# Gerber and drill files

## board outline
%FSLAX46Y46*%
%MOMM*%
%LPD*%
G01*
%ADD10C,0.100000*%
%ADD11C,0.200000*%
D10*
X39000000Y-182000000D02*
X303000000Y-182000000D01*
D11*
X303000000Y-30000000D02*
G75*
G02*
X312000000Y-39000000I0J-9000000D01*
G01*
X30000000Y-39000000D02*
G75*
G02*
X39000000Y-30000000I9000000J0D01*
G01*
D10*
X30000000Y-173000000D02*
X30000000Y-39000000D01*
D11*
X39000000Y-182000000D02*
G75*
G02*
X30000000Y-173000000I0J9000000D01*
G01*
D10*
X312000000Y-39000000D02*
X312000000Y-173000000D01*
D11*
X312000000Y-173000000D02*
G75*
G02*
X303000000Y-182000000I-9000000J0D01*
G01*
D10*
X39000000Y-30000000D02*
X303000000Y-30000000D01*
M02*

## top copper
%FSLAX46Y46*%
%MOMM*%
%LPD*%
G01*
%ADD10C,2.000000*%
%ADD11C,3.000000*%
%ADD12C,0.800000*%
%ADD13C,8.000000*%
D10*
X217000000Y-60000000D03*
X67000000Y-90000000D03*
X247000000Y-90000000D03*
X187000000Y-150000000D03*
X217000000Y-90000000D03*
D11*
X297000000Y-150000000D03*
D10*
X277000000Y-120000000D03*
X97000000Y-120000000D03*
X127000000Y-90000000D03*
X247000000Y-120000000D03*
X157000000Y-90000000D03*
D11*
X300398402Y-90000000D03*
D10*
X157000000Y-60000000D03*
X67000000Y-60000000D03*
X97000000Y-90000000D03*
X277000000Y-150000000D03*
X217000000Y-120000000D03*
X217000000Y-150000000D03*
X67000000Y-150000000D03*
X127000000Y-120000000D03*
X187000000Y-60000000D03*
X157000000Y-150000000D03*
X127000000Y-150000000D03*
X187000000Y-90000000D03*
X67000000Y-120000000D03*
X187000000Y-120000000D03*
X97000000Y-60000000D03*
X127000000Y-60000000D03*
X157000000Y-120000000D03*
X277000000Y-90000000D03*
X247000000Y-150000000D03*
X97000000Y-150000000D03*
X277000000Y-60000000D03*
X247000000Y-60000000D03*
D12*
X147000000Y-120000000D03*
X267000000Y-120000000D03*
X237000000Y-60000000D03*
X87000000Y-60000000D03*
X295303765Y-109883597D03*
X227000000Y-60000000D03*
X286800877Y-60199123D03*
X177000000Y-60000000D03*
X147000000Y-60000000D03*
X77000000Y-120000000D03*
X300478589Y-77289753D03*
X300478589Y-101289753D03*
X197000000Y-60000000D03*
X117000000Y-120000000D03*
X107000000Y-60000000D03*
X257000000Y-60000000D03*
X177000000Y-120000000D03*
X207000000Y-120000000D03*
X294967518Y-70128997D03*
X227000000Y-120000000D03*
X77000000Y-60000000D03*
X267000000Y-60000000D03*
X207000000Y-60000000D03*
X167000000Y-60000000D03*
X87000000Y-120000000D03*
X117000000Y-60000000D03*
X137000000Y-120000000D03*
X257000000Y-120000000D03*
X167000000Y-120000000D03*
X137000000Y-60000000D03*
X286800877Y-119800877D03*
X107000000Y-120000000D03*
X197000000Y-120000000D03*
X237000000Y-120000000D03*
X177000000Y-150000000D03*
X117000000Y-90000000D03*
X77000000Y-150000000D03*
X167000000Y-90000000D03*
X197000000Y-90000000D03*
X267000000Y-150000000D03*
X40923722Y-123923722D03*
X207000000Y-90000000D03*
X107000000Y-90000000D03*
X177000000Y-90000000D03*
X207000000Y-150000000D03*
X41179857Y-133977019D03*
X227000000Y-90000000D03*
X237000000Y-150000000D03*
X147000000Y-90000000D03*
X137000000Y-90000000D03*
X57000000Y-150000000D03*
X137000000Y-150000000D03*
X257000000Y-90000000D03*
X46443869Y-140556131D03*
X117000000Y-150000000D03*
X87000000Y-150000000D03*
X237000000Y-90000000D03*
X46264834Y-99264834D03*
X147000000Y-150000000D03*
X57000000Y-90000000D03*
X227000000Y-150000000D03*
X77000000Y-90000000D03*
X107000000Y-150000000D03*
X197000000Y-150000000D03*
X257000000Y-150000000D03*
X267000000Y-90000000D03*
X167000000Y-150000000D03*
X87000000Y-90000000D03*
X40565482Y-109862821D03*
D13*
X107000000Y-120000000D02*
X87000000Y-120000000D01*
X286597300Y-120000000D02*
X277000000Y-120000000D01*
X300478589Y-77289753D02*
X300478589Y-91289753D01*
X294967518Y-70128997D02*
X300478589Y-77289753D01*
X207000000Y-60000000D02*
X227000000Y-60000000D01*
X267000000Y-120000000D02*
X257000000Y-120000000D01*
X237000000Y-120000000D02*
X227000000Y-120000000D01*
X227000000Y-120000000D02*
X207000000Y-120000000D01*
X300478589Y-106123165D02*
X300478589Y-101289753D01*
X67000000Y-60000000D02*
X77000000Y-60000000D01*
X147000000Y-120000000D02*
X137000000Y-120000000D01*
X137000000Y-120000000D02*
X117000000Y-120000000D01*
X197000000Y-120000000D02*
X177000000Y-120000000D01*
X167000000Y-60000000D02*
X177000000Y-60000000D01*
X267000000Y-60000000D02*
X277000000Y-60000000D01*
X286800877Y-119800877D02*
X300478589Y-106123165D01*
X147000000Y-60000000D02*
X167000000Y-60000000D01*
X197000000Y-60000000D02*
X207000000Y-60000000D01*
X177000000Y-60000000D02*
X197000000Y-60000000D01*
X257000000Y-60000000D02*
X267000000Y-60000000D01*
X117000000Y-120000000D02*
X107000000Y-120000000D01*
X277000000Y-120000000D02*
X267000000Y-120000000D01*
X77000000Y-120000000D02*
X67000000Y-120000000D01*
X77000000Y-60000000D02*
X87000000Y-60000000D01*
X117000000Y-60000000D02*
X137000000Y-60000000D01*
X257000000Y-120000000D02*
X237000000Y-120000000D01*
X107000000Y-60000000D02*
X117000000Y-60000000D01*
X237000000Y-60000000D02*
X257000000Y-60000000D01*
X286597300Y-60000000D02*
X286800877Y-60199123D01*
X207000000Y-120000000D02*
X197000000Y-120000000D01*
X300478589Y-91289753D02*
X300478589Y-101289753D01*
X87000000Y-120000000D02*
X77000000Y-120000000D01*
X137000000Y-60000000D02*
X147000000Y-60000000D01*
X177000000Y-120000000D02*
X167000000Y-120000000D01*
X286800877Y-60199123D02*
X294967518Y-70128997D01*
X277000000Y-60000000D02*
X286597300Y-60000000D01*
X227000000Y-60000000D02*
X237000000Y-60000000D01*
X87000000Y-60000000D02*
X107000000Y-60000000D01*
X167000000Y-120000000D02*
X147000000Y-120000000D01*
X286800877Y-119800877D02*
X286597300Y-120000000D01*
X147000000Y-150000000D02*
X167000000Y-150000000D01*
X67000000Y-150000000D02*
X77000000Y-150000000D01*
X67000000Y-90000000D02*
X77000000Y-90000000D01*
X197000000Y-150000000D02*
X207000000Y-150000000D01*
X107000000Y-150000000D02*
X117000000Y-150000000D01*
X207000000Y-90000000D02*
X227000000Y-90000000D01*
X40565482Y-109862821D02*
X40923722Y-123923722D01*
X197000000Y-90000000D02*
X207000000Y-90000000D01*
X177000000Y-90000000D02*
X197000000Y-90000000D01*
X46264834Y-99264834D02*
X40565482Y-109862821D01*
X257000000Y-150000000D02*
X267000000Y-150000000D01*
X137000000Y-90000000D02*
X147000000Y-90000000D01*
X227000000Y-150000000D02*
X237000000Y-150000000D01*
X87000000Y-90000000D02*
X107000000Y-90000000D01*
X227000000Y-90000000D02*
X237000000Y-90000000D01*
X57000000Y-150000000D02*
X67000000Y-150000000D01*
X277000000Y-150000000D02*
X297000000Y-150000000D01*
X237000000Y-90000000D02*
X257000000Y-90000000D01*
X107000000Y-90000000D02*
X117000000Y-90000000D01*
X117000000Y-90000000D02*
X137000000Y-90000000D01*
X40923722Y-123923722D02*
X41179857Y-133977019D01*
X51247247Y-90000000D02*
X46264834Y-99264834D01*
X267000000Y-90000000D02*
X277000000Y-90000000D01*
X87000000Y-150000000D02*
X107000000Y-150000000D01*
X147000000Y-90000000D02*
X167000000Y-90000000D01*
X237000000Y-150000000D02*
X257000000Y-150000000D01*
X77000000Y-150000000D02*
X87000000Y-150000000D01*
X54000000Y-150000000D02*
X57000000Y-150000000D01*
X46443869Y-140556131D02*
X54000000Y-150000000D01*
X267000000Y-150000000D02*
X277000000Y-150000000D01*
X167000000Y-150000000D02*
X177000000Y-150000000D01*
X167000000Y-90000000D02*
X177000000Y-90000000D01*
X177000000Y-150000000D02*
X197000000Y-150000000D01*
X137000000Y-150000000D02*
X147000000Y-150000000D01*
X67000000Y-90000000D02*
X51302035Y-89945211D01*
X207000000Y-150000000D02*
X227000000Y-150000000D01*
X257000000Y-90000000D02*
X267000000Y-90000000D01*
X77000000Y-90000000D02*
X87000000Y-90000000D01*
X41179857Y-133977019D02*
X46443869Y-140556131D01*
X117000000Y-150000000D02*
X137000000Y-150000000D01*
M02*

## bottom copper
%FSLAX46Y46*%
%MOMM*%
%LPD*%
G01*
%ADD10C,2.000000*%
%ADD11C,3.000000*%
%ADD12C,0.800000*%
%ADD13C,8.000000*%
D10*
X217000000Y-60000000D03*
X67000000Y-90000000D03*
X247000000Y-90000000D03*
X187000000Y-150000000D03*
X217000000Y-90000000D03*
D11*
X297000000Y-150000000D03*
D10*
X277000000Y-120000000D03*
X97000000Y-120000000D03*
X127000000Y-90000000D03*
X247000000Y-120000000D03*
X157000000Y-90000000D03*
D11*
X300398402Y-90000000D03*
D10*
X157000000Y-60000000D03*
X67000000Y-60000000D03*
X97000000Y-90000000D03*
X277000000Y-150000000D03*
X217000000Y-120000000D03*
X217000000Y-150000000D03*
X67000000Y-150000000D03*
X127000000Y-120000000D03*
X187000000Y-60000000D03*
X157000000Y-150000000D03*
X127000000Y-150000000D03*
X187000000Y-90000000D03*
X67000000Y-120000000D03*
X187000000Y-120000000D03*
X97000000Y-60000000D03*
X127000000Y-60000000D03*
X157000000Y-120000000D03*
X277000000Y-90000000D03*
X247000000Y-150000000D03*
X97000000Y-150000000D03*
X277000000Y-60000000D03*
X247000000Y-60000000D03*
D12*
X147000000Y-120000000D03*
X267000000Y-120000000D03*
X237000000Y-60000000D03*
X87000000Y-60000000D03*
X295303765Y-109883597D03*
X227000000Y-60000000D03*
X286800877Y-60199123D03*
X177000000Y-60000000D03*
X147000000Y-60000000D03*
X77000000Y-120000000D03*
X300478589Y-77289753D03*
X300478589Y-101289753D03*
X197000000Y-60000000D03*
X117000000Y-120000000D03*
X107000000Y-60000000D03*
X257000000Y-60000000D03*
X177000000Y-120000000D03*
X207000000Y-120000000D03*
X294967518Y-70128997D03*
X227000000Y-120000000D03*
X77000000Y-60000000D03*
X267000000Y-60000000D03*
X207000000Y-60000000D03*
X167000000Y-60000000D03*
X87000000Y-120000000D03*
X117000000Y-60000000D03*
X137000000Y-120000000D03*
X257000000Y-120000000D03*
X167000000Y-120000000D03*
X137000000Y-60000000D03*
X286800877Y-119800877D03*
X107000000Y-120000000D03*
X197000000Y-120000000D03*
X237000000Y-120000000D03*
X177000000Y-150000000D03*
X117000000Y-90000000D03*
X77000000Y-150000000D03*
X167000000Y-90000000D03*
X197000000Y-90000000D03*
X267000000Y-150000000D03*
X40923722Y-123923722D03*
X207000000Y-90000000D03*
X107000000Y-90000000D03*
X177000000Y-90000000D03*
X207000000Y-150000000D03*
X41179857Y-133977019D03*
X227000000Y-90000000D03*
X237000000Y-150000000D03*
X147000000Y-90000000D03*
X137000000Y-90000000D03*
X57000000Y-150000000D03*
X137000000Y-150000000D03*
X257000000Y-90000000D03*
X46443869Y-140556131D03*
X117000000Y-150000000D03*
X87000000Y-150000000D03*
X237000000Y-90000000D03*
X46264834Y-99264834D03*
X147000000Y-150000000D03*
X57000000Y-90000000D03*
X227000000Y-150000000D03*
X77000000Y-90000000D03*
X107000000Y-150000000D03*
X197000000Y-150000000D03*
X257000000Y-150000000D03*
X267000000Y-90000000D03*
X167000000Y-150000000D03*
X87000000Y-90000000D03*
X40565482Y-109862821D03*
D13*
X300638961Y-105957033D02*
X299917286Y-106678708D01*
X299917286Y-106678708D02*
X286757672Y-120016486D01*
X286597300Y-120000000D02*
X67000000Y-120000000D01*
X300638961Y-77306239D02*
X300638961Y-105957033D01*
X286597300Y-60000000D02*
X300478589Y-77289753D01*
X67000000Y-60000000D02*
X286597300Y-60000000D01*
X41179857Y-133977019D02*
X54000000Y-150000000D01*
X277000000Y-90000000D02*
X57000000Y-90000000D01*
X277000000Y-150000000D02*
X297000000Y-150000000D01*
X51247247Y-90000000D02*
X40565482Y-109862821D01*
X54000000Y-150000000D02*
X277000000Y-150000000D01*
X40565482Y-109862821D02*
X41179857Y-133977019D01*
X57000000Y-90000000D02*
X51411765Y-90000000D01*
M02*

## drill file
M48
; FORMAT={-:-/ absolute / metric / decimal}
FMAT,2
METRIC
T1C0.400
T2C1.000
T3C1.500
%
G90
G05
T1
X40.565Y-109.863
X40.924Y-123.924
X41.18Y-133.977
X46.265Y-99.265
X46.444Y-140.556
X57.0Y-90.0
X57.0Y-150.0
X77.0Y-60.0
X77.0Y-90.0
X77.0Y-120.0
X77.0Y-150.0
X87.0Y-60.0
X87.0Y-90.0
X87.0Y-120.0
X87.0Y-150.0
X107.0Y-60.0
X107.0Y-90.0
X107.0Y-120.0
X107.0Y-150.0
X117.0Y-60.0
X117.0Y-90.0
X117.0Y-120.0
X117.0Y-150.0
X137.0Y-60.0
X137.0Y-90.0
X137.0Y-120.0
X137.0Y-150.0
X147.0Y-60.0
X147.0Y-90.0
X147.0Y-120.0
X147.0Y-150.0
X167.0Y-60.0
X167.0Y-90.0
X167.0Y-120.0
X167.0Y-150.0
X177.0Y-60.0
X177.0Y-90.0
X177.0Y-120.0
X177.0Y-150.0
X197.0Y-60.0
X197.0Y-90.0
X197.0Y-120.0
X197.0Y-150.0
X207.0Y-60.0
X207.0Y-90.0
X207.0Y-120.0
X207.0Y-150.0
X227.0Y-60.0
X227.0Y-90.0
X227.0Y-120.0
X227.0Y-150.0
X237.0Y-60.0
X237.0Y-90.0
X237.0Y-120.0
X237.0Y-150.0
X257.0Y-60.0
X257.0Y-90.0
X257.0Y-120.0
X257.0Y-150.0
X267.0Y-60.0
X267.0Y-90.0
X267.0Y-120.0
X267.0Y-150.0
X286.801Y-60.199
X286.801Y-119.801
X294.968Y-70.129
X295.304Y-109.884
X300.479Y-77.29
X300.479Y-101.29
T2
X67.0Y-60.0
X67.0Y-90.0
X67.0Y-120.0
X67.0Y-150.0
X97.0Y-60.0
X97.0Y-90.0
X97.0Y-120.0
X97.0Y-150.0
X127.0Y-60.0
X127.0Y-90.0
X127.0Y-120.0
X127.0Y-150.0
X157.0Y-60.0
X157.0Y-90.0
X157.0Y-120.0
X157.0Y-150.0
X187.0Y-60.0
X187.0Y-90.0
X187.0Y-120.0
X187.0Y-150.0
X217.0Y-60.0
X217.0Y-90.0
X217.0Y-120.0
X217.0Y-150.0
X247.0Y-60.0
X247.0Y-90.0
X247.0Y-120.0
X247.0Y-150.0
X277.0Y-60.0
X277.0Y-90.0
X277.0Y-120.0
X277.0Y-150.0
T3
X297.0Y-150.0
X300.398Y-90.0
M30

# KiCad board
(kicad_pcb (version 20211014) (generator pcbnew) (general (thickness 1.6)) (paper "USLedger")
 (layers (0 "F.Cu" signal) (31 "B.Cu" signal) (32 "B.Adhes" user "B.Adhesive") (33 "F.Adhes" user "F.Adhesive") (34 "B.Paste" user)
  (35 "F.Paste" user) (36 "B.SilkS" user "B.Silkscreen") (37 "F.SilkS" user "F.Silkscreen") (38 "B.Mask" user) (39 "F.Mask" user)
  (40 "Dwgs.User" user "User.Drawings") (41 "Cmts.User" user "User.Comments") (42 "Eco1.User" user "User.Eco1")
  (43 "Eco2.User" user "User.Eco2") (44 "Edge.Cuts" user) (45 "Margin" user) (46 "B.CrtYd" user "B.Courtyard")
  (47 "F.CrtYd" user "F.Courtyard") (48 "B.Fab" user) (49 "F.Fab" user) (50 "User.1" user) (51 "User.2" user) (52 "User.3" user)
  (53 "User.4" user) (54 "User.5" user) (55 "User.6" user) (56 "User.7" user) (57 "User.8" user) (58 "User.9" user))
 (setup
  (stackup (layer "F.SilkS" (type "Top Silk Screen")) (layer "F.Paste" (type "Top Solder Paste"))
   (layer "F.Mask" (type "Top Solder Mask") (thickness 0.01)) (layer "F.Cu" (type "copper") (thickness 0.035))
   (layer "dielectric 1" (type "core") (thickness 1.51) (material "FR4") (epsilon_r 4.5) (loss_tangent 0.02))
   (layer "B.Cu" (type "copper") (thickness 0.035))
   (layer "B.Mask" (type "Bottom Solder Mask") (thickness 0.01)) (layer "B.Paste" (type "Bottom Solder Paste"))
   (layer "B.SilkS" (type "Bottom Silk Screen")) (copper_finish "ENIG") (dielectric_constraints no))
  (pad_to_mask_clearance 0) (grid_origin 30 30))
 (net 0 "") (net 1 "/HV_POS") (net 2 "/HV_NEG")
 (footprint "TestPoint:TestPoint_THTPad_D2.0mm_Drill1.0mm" (layer "F.Cu") (at 217 60)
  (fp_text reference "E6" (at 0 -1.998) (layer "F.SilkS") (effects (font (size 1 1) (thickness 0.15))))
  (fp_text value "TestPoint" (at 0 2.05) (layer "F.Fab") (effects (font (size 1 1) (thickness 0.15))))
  (pad "1" thru_hole circle (at 0 0) (size 2 2) (drill 1) (layers *.Cu *.Mask) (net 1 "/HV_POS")))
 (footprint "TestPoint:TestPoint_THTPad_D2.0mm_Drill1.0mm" (layer "F.Cu") (at 67 90)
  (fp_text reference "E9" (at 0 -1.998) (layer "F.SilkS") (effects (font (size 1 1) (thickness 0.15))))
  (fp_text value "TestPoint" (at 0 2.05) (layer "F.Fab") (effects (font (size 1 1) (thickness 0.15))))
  (pad "1" thru_hole circle (at 0 0) (size 2 2) (drill 1) (layers *.Cu *.Mask) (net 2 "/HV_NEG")))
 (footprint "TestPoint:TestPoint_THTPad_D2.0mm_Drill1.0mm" (layer "F.Cu") (at 247 90)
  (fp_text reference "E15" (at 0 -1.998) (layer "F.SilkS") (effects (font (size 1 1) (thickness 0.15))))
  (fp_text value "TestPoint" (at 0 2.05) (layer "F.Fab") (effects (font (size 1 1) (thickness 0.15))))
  (pad "1" thru_hole circle (at 0 0) (size 2 2) (drill 1) (layers *.Cu *.Mask) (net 2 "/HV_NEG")))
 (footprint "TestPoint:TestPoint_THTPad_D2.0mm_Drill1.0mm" (layer "F.Cu") (at 187 150)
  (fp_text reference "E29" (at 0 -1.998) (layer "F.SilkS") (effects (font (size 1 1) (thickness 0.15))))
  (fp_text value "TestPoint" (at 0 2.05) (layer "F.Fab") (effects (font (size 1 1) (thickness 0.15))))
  (pad "1" thru_hole circle (at 0 0) (size 2 2) (drill 1) (layers *.Cu *.Mask) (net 2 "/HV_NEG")))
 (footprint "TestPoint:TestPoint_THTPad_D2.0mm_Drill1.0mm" (layer "F.Cu") (at 217 90)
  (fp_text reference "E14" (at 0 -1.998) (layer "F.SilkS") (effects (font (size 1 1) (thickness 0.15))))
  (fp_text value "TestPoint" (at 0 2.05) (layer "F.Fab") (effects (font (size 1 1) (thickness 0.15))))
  (pad "1" thru_hole circle (at 0 0) (size 2 2) (drill 1) (layers *.Cu *.Mask) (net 2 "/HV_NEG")))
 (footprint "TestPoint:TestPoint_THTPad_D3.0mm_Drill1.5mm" (layer "F.Cu") (at 297 150)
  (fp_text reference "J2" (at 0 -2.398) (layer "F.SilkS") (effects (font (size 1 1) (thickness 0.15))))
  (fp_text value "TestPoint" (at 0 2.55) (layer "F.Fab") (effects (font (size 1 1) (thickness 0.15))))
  (pad "1" thru_hole circle (at 0 0) (size 3 3) (drill 1.5) (layers *.Cu *.Mask) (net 2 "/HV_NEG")))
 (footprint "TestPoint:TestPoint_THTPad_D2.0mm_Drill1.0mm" (layer "F.Cu") (at 277 120)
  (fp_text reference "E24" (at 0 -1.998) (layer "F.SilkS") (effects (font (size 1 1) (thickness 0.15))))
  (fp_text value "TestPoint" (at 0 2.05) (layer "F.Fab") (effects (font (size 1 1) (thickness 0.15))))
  (pad "1" thru_hole circle (at 0 0) (size 2 2) (drill 1) (layers *.Cu *.Mask) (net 1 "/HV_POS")))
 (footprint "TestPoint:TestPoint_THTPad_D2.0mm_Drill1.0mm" (layer "F.Cu") (at 97 120)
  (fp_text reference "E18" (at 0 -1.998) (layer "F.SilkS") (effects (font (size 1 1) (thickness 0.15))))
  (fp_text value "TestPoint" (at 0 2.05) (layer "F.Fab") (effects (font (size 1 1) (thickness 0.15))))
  (pad "1" thru_hole circle (at 0 0) (size 2 2) (drill 1) (layers *.Cu *.Mask) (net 1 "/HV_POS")))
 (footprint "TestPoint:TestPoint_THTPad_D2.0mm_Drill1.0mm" (layer "F.Cu") (at 127 90)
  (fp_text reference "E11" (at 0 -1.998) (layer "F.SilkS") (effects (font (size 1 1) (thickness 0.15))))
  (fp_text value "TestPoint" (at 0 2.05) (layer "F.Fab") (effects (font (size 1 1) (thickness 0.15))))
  (pad "1" thru_hole circle (at 0 0) (size 2 2) (drill 1) (layers *.Cu *.Mask) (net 2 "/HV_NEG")))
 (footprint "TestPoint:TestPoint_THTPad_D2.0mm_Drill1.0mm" (layer "F.Cu") (at 247 120)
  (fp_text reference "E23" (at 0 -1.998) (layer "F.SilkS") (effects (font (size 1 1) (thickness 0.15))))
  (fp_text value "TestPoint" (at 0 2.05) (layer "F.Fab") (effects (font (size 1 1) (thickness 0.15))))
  (pad "1" thru_hole circle (at 0 0) (size 2 2) (drill 1) (layers *.Cu *.Mask) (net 1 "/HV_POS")))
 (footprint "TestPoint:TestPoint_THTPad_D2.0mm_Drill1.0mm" (layer "F.Cu") (at 157 90)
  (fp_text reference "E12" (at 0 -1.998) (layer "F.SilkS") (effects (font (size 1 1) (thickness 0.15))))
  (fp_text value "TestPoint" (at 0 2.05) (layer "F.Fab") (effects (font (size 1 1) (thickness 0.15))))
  (pad "1" thru_hole circle (at 0 0) (size 2 2) (drill 1) (layers *.Cu *.Mask) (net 2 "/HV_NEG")))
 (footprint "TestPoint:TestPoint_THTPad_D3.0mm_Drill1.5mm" (layer "F.Cu") (at 300.398402 90)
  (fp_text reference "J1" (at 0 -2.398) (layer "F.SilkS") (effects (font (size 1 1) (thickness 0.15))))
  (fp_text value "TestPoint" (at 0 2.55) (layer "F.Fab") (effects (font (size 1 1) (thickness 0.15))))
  (pad "1" thru_hole circle (at 0 0) (size 3 3) (drill 1.5) (layers *.Cu *.Mask) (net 1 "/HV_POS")))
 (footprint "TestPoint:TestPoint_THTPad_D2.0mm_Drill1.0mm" (layer "F.Cu") (at 157 60)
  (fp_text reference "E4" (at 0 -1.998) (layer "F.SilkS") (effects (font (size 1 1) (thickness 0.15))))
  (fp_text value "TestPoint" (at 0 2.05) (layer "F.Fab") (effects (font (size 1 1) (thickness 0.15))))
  (pad "1" thru_hole circle (at 0 0) (size 2 2) (drill 1) (layers *.Cu *.Mask) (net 1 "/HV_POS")))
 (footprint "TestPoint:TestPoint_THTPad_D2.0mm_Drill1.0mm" (layer "F.Cu") (at 67 60)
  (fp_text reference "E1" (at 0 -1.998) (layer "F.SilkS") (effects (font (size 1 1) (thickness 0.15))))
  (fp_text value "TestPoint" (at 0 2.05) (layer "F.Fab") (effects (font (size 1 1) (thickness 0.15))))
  (pad "1" thru_hole circle (at 0 0) (size 2 2) (drill 1) (layers *.Cu *.Mask) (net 1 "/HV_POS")))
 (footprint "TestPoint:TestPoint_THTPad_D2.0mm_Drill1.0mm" (layer "F.Cu") (at 97 90)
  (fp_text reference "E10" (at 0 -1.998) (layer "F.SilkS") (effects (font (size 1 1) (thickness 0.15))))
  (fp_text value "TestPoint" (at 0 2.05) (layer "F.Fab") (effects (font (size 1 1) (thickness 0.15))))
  (pad "1" thru_hole circle (at 0 0) (size 2 2) (drill 1) (layers *.Cu *.Mask) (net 2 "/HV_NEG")))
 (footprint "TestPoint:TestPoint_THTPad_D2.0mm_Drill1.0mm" (layer "F.Cu") (at 277 150)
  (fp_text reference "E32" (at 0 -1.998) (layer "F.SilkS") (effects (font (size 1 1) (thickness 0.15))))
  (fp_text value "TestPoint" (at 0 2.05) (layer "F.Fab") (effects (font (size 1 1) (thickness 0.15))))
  (pad "1" thru_hole circle (at 0 0) (size 2 2) (drill 1) (layers *.Cu *.Mask) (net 2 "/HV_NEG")))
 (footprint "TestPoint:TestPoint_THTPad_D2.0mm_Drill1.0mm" (layer "F.Cu") (at 217 120)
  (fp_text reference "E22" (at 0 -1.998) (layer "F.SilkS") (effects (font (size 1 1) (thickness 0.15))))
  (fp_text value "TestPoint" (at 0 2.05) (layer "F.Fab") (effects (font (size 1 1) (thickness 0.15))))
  (pad "1" thru_hole circle (at 0 0) (size 2 2) (drill 1) (layers *.Cu *.Mask) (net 1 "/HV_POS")))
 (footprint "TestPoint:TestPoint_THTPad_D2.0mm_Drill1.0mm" (layer "F.Cu") (at 217 150)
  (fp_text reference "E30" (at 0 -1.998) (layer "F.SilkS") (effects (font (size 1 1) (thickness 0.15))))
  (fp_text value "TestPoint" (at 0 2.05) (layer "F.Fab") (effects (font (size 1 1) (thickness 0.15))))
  (pad "1" thru_hole circle (at 0 0) (size 2 2) (drill 1) (layers *.Cu *.Mask) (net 2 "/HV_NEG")))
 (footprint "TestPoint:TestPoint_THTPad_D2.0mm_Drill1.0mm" (layer "F.Cu") (at 67 150)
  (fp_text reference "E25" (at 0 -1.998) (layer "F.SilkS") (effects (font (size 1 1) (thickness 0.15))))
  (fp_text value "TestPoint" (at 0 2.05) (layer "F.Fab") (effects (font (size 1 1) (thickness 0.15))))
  (pad "1" thru_hole circle (at 0 0) (size 2 2) (drill 1) (layers *.Cu *.Mask) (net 2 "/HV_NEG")))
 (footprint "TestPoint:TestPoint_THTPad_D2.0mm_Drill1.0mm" (layer "F.Cu") (at 127 120)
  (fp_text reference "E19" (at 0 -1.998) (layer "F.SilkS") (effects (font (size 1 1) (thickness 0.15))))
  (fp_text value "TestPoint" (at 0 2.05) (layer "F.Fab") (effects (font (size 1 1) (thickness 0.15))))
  (pad "1" thru_hole circle (at 0 0) (size 2 2) (drill 1) (layers *.Cu *.Mask) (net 1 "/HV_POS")))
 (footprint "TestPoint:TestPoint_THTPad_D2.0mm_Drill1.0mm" (layer "F.Cu") (at 187 60)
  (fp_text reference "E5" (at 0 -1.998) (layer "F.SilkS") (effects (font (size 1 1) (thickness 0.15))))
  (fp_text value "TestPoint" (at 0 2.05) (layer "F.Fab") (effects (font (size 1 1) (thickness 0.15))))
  (pad "1" thru_hole circle (at 0 0) (size 2 2) (drill 1) (layers *.Cu *.Mask) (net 1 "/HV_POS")))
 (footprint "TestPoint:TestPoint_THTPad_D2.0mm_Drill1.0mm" (layer "F.Cu") (at 157 150)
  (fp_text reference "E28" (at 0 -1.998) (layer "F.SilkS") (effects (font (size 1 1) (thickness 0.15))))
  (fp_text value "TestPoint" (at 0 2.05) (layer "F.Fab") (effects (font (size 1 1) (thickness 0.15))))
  (pad "1" thru_hole circle (at 0 0) (size 2 2) (drill 1) (layers *.Cu *.Mask) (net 2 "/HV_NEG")))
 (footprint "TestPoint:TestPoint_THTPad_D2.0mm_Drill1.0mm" (layer "F.Cu") (at 127 150)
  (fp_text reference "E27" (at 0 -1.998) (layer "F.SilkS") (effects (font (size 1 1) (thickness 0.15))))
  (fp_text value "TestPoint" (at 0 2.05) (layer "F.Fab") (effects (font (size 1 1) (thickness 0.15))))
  (pad "1" thru_hole circle (at 0 0) (size 2 2) (drill 1) (layers *.Cu *.Mask) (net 2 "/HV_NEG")))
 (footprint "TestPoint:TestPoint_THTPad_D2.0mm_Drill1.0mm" (layer "F.Cu") (at 187 90)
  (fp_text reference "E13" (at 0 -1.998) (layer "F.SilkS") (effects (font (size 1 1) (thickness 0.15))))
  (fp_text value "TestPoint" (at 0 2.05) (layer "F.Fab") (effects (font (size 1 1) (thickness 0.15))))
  (pad "1" thru_hole circle (at 0 0) (size 2 2) (drill 1) (layers *.Cu *.Mask) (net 2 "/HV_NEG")))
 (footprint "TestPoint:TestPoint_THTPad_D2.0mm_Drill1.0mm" (layer "F.Cu") (at 67 120)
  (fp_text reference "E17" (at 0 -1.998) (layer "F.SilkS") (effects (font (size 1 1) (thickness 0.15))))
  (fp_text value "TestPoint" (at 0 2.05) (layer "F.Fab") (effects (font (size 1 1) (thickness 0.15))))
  (pad "1" thru_hole circle (at 0 0) (size 2 2) (drill 1) (layers *.Cu *.Mask) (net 1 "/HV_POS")))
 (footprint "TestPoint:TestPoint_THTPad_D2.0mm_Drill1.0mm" (layer "F.Cu") (at 187 120)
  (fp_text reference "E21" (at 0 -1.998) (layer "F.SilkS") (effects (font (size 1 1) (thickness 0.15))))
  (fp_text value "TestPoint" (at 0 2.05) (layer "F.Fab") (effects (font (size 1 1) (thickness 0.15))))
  (pad "1" thru_hole circle (at 0 0) (size 2 2) (drill 1) (layers *.Cu *.Mask) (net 1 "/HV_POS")))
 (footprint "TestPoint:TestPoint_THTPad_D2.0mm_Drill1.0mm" (layer "F.Cu") (at 97 60)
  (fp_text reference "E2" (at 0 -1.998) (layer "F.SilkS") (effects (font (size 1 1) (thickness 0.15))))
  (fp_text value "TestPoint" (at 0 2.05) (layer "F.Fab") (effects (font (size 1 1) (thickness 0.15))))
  (pad "1" thru_hole circle (at 0 0) (size 2 2) (drill 1) (layers *.Cu *.Mask) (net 1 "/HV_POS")))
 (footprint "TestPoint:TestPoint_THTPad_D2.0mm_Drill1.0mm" (layer "F.Cu") (at 127 60)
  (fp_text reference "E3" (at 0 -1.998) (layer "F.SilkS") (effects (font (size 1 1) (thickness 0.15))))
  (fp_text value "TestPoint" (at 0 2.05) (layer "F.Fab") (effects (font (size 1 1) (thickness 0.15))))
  (pad "1" thru_hole circle (at 0 0) (size 2 2) (drill 1) (layers *.Cu *.Mask) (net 1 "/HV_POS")))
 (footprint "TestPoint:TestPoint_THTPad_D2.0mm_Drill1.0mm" (layer "F.Cu") (at 157 120)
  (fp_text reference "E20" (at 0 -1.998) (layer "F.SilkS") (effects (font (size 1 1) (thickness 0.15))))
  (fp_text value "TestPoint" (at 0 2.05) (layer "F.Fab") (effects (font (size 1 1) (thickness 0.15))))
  (pad "1" thru_hole circle (at 0 0) (size 2 2) (drill 1) (layers *.Cu *.Mask) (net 1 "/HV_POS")))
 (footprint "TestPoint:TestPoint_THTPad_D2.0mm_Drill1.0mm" (layer "F.Cu") (at 277 90)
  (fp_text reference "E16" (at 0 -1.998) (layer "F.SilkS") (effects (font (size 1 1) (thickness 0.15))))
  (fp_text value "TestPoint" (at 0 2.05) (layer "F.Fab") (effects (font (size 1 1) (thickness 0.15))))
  (pad "1" thru_hole circle (at 0 0) (size 2 2) (drill 1) (layers *.Cu *.Mask) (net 2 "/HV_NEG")))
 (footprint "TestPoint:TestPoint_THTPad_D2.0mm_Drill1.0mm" (layer "F.Cu") (at 247 150)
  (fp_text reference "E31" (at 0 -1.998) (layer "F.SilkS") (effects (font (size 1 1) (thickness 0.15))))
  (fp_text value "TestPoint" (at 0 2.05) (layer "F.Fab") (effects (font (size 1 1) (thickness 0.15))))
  (pad "1" thru_hole circle (at 0 0) (size 2 2) (drill 1) (layers *.Cu *.Mask) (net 2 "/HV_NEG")))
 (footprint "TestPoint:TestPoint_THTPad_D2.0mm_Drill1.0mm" (layer "F.Cu") (at 97 150)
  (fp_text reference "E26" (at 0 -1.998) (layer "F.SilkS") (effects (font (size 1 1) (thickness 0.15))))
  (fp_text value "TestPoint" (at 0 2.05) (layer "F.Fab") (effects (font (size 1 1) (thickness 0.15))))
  (pad "1" thru_hole circle (at 0 0) (size 2 2) (drill 1) (layers *.Cu *.Mask) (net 2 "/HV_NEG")))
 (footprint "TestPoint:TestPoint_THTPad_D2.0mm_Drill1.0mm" (layer "F.Cu") (at 277 60)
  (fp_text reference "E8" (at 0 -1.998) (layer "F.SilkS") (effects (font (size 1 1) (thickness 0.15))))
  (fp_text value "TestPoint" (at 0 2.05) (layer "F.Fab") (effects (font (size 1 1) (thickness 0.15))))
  (pad "1" thru_hole circle (at 0 0) (size 2 2) (drill 1) (layers *.Cu *.Mask) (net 1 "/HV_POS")))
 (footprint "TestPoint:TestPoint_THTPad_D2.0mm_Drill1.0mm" (layer "F.Cu") (at 247 60)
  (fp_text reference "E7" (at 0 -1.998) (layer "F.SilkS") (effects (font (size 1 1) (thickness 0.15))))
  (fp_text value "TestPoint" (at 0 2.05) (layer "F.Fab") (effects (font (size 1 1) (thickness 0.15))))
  (pad "1" thru_hole circle (at 0 0) (size 2 2) (drill 1) (layers *.Cu *.Mask) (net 1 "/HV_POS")))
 (gr_line (start 39 182) (end 303 182) (layer "Edge.Cuts") (width 0.1))
 (gr_arc (start 303 30) (mid 309.363961 32.636039) (end 312 39) (layer "Edge.Cuts") (width 0.2))
 (gr_arc (start 30 39) (mid 32.636039 32.636039) (end 39 30) (layer "Edge.Cuts") (width 0.2))
 (gr_line (start 30 173) (end 30 39) (layer "Edge.Cuts") (width 0.1))
 (gr_arc (start 39 182) (mid 32.636039 179.363961) (end 30 173) (layer "Edge.Cuts") (width 0.2))
 (gr_line (start 312 39) (end 312 173) (layer "Edge.Cuts") (width 0.1))
 (gr_arc (start 312 173) (mid 309.363961 179.363961) (end 303 182) (layer "Edge.Cuts") (width 0.2))
 (gr_line (start 39 30) (end 303 30) (layer "Edge.Cuts") (width 0.1))
 (segment (start 107 120) (end 87 120) (width 8) (layer "F.Cu") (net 1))
 (segment (start 286.5973 120) (end 277 120) (width 8) (layer "F.Cu") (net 1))
 (segment (start 300.478589 77.289753) (end 300.478589 91.289753) (width 8) (layer "F.Cu") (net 1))
 (segment (start 294.967518 70.128997) (end 300.478589 77.289753) (width 8) (layer "F.Cu") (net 1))
 (segment (start 207 60) (end 227 60) (width 8) (layer "F.Cu") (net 1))
 (segment (start 267 120) (end 257 120) (width 8) (layer "F.Cu") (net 1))
 (segment (start 237 120) (end 227 120) (width 8) (layer "F.Cu") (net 1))
 (segment (start 227 120) (end 207 120) (width 8) (layer "F.Cu") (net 1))
 (segment (start 300.478589 106.123165) (end 300.478589 101.289753) (width 8) (layer "F.Cu") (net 1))
 (segment (start 67 60) (end 77 60) (width 8) (layer "F.Cu") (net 1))
 (segment (start 147 120) (end 137 120) (width 8) (layer "F.Cu") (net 1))
 (segment (start 137 120) (end 117 120) (width 8) (layer "F.Cu") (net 1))
 (segment (start 197 120) (end 177 120) (width 8) (layer "F.Cu") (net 1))
 (segment (start 167 60) (end 177 60) (width 8) (layer "F.Cu") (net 1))
 (segment (start 267 60) (end 277 60) (width 8) (layer "F.Cu") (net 1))
 (segment (start 286.800877 119.800877) (end 300.478589 106.123165) (width 8) (layer "F.Cu") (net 1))
 (segment (start 147 60) (end 167 60) (width 8) (layer "F.Cu") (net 1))
 (segment (start 197 60) (end 207 60) (width 8) (layer "F.Cu") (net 1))
 (segment (start 177 60) (end 197 60) (width 8) (layer "F.Cu") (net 1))
 (segment (start 257 60) (end 267 60) (width 8) (layer "F.Cu") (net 1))
 (segment (start 117 120) (end 107 120) (width 8) (layer "F.Cu") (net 1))
 (segment (start 277 120) (end 267 120) (width 8) (layer "F.Cu") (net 1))
 (segment (start 77 120) (end 67 120) (width 8) (layer "F.Cu") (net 1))
 (segment (start 77 60) (end 87 60) (width 8) (layer "F.Cu") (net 1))
 (segment (start 117 60) (end 137 60) (width 8) (layer "F.Cu") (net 1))
 (segment (start 257 120) (end 237 120) (width 8) (layer "F.Cu") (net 1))
 (segment (start 107 60) (end 117 60) (width 8) (layer "F.Cu") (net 1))
 (segment (start 237 60) (end 257 60) (width 8) (layer "F.Cu") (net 1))
 (segment (start 286.5973 60) (end 286.800877 60.199123) (width 8) (layer "F.Cu") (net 1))
 (segment (start 207 120) (end 197 120) (width 8) (layer "F.Cu") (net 1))
 (segment (start 300.478589 91.289753) (end 300.478589 101.289753) (width 8) (layer "F.Cu") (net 1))
 (segment (start 87 120) (end 77 120) (width 8) (layer "F.Cu") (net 1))
 (segment (start 137 60) (end 147 60) (width 8) (layer "F.Cu") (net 1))
 (segment (start 177 120) (end 167 120) (width 8) (layer "F.Cu") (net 1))
 (segment (start 286.800877 60.199123) (end 294.967518 70.128997) (width 8) (layer "F.Cu") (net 1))
 (segment (start 277 60) (end 286.5973 60) (width 8) (layer "F.Cu") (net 1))
 (segment (start 227 60) (end 237 60) (width 8) (layer "F.Cu") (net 1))
 (segment (start 87 60) (end 107 60) (width 8) (layer "F.Cu") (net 1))
 (segment (start 167 120) (end 147 120) (width 8) (layer "F.Cu") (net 1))
 (segment (start 286.800877 119.800877) (end 286.5973 120) (width 8) (layer "F.Cu") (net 1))
 (via (at 147 120) (size 0.8) (drill 0.4) (layers "F.Cu" "B.Cu") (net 1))
 (via (at 267 120) (size 0.8) (drill 0.4) (layers "F.Cu" "B.Cu") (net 1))
 (via (at 237 60) (size 0.8) (drill 0.4) (layers "F.Cu" "B.Cu") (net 1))
 (via (at 87 60) (size 0.8) (drill 0.4) (layers "F.Cu" "B.Cu") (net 1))
 (via (at 295.303765 109.883597) (size 0.8) (drill 0.4) (layers "F.Cu" "B.Cu") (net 1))
 (via (at 227 60) (size 0.8) (drill 0.4) (layers "F.Cu" "B.Cu") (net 1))
 (via (at 286.800877 60.199123) (size 0.8) (drill 0.4) (layers "F.Cu" "B.Cu") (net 1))
 (via (at 177 60) (size 0.8) (drill 0.4) (layers "F.Cu" "B.Cu") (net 1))
 (via (at 147 60) (size 0.8) (drill 0.4) (layers "F.Cu" "B.Cu") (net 1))
 (via (at 77 120) (size 0.8) (drill 0.4) (layers "F.Cu" "B.Cu") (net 1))
 (via (at 300.478589 77.289753) (size 0.8) (drill 0.4) (layers "F.Cu" "B.Cu") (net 1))
 (via (at 300.478589 101.289753) (size 0.8) (drill 0.4) (layers "F.Cu" "B.Cu") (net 1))
 (via (at 197 60) (size 0.8) (drill 0.4) (layers "F.Cu" "B.Cu") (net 1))
 (via (at 117 120) (size 0.8) (drill 0.4) (layers "F.Cu" "B.Cu") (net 1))
 (via (at 107 60) (size 0.8) (drill 0.4) (layers "F.Cu" "B.Cu") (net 1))
 (via (at 257 60) (size 0.8) (drill 0.4) (layers "F.Cu" "B.Cu") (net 1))
 (via (at 177 120) (size 0.8) (drill 0.4) (layers "F.Cu" "B.Cu") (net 1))
 (via (at 207 120) (size 0.8) (drill 0.4) (layers "F.Cu" "B.Cu") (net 1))
 (via (at 294.967518 70.128997) (size 0.8) (drill 0.4) (layers "F.Cu" "B.Cu") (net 1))
 (via (at 227 120) (size 0.8) (drill 0.4) (layers "F.Cu" "B.Cu") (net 1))
 (via (at 77 60) (size 0.8) (drill 0.4) (layers "F.Cu" "B.Cu") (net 1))
 (via (at 267 60) (size 0.8) (drill 0.4) (layers "F.Cu" "B.Cu") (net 1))
 (via (at 207 60) (size 0.8) (drill 0.4) (layers "F.Cu" "B.Cu") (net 1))
 (via (at 167 60) (size 0.8) (drill 0.4) (layers "F.Cu" "B.Cu") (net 1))
 (via (at 87 120) (size 0.8) (drill 0.4) (layers "F.Cu" "B.Cu") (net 1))
 (via (at 117 60) (size 0.8) (drill 0.4) (layers "F.Cu" "B.Cu") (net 1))
 (via (at 137 120) (size 0.8) (drill 0.4) (layers "F.Cu" "B.Cu") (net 1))
 (via (at 257 120) (size 0.8) (drill 0.4) (layers "F.Cu" "B.Cu") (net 1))
 (via (at 167 120) (size 0.8) (drill 0.4) (layers "F.Cu" "B.Cu") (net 1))
 (via (at 137 60) (size 0.8) (drill 0.4) (layers "F.Cu" "B.Cu") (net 1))
 (via (at 286.800877 119.800877) (size 0.8) (drill 0.4) (layers "F.Cu" "B.Cu") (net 1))
 (via (at 107 120) (size 0.8) (drill 0.4) (layers "F.Cu" "B.Cu") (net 1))
 (via (at 197 120) (size 0.8) (drill 0.4) (layers "F.Cu" "B.Cu") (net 1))
 (via (at 237 120) (size 0.8) (drill 0.4) (layers "F.Cu" "B.Cu") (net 1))
 (segment (start 300.638961 105.957033) (end 299.917286 106.678708) (width 8) (layer "B.Cu") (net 1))
 (segment (start 299.917286 106.678708) (end 286.757672 120.016486) (width 8) (layer "B.Cu") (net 1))
 (segment (start 286.5973 120) (end 67 120) (width 8) (layer "B.Cu") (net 1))
 (segment (start 300.638961 77.306239) (end 300.638961 105.957033) (width 8) (layer "B.Cu") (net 1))
 (segment (start 286.5973 60) (end 300.478589 77.289753) (width 8) (layer "B.Cu") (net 1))
 (segment (start 67 60) (end 286.5973 60) (width 8) (layer "B.Cu") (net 1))
 (segment (start 147 150) (end 167 150) (width 8) (layer "F.Cu") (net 2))
 (segment (start 67 150) (end 77 150) (width 8) (layer "F.Cu") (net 2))
 (segment (start 67 90) (end 77 90) (width 8) (layer "F.Cu") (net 2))
 (segment (start 197 150) (end 207 150) (width 8) (layer "F.Cu") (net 2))
 (segment (start 107 150) (end 117 150) (width 8) (layer "F.Cu") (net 2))
 (segment (start 207 90) (end 227 90) (width 8) (layer "F.Cu") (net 2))
 (segment (start 40.565482 109.862821) (end 40.923722 123.923722) (width 8) (layer "F.Cu") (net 2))
 (segment (start 197 90) (end 207 90) (width 8) (layer "F.Cu") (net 2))
 (segment (start 177 90) (end 197 90) (width 8) (layer "F.Cu") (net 2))
 (segment (start 46.264834 99.264834) (end 40.565482 109.862821) (width 8) (layer "F.Cu") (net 2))
 (segment (start 257 150) (end 267 150) (width 8) (layer "F.Cu") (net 2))
 (segment (start 137 90) (end 147 90) (width 8) (layer "F.Cu") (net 2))
 (segment (start 227 150) (end 237 150) (width 8) (layer "F.Cu") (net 2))
 (segment (start 87 90) (end 107 90) (width 8) (layer "F.Cu") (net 2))
 (segment (start 227 90) (end 237 90) (width 8) (layer "F.Cu") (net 2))
 (segment (start 57 150) (end 67 150) (width 8) (layer "F.Cu") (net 2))
 (segment (start 277 150) (end 297 150) (width 8) (layer "F.Cu") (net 2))
 (segment (start 237 90) (end 257 90) (width 8) (layer "F.Cu") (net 2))
 (segment (start 107 90) (end 117 90) (width 8) (layer "F.Cu") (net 2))
 (segment (start 117 90) (end 137 90) (width 8) (layer "F.Cu") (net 2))
 (segment (start 40.923722 123.923722) (end 41.179857 133.977019) (width 8) (layer "F.Cu") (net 2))
 (segment (start 51.247247 90) (end 46.264834 99.264834) (width 8) (layer "F.Cu") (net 2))
 (segment (start 267 90) (end 277 90) (width 8) (layer "F.Cu") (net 2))
 (segment (start 87 150) (end 107 150) (width 8) (layer "F.Cu") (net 2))
 (segment (start 147 90) (end 167 90) (width 8) (layer "F.Cu") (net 2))
 (segment (start 237 150) (end 257 150) (width 8) (layer "F.Cu") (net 2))
 (segment (start 77 150) (end 87 150) (width 8) (layer "F.Cu") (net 2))
 (segment (start 54 150) (end 57 150) (width 8) (layer "F.Cu") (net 2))
 (segment (start 46.443869 140.556131) (end 54 150) (width 8) (layer "F.Cu") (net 2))
 (segment (start 267 150) (end 277 150) (width 8) (layer "F.Cu") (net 2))
 (segment (start 167 150) (end 177 150) (width 8) (layer "F.Cu") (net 2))
 (segment (start 167 90) (end 177 90) (width 8) (layer "F.Cu") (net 2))
 (segment (start 177 150) (end 197 150) (width 8) (layer "F.Cu") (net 2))
 (segment (start 137 150) (end 147 150) (width 8) (layer "F.Cu") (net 2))
 (segment (start 67 90) (end 51.302035 89.945211) (width 8) (layer "F.Cu") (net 2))
 (segment (start 207 150) (end 227 150) (width 8) (layer "F.Cu") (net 2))
 (segment (start 257 90) (end 267 90) (width 8) (layer "F.Cu") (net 2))
 (segment (start 77 90) (end 87 90) (width 8) (layer "F.Cu") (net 2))
 (segment (start 41.179857 133.977019) (end 46.443869 140.556131) (width 8) (layer "F.Cu") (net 2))
 (segment (start 117 150) (end 137 150) (width 8) (layer "F.Cu") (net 2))
 (via (at 177 150) (size 0.8) (drill 0.4) (layers "F.Cu" "B.Cu") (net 2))
 (via (at 117 90) (size 0.8) (drill 0.4) (layers "F.Cu" "B.Cu") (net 2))
 (via (at 77 150) (size 0.8) (drill 0.4) (layers "F.Cu" "B.Cu") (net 2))
 (via (at 167 90) (size 0.8) (drill 0.4) (layers "F.Cu" "B.Cu") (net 2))
 (via (at 197 90) (size 0.8) (drill 0.4) (layers "F.Cu" "B.Cu") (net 2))
 (via (at 267 150) (size 0.8) (drill 0.4) (layers "F.Cu" "B.Cu") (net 2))
 (via (at 40.923722 123.923722) (size 0.8) (drill 0.4) (layers "F.Cu" "B.Cu") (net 2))
 (via (at 207 90) (size 0.8) (drill 0.4) (layers "F.Cu" "B.Cu") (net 2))
 (via (at 107 90) (size 0.8) (drill 0.4) (layers "F.Cu" "B.Cu") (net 2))
 (via (at 177 90) (size 0.8) (drill 0.4) (layers "F.Cu" "B.Cu") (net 2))
 (via (at 207 150) (size 0.8) (drill 0.4) (layers "F.Cu" "B.Cu") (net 2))
 (via (at 41.179857 133.977019) (size 0.8) (drill 0.4) (layers "F.Cu" "B.Cu") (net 2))
 (via (at 227 90) (size 0.8) (drill 0.4) (layers "F.Cu" "B.Cu") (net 2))
 (via (at 237 150) (size 0.8) (drill 0.4) (layers "F.Cu" "B.Cu") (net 2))
 (via (at 147 90) (size 0.8) (drill 0.4) (layers "F.Cu" "B.Cu") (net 2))
 (via (at 137 90) (size 0.8) (drill 0.4) (layers "F.Cu" "B.Cu") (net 2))
 (via (at 57 150) (size 0.8) (drill 0.4) (layers "F.Cu" "B.Cu") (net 2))
 (via (at 137 150) (size 0.8) (drill 0.4) (layers "F.Cu" "B.Cu") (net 2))
 (via (at 257 90) (size 0.8) (drill 0.4) (layers "F.Cu" "B.Cu") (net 2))
 (via (at 46.443869 140.556131) (size 0.8) (drill 0.4) (layers "F.Cu" "B.Cu") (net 2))
 (via (at 117 150) (size 0.8) (drill 0.4) (layers "F.Cu" "B.Cu") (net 2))
 (via (at 87 150) (size 0.8) (drill 0.4) (layers "F.Cu" "B.Cu") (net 2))
 (via (at 237 90) (size 0.8) (drill 0.4) (layers "F.Cu" "B.Cu") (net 2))
 (via (at 46.264834 99.264834) (size 0.8) (drill 0.4) (layers "F.Cu" "B.Cu") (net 2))
 (via (at 147 150) (size 0.8) (drill 0.4) (layers "F.Cu" "B.Cu") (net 2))
 (via (at 57 90) (size 0.8) (drill 0.4) (layers "F.Cu" "B.Cu") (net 2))
 (via (at 227 150) (size 0.8) (drill 0.4) (layers "F.Cu" "B.Cu") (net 2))
 (via (at 77 90) (size 0.8) (drill 0.4) (layers "F.Cu" "B.Cu") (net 2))
 (via (at 107 150) (size 0.8) (drill 0.4) (layers "F.Cu" "B.Cu") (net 2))
 (via (at 197 150) (size 0.8) (drill 0.4) (layers "F.Cu" "B.Cu") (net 2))
 (via (at 257 150) (size 0.8) (drill 0.4) (layers "F.Cu" "B.Cu") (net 2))
 (via (at 267 90) (size 0.8) (drill 0.4) (layers "F.Cu" "B.Cu") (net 2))
 (via (at 167 150) (size 0.8) (drill 0.4) (layers "F.Cu" "B.Cu") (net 2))
 (via (at 87 90) (size 0.8) (drill 0.4) (layers "F.Cu" "B.Cu") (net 2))
 (via (at 40.565482 109.862821) (size 0.8) (drill 0.4) (layers "F.Cu" "B.Cu") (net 2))
 (segment (start 41.179857 133.977019) (end 54 150) (width 8) (layer "B.Cu") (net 2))
 (segment (start 277 90) (end 57 90) (width 8) (layer "B.Cu") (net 2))
 (segment (start 277 150) (end 297 150) (width 8) (layer "B.Cu") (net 2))
 (segment (start 51.247247 90) (end 40.565482 109.862821) (width 8) (layer "B.Cu") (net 2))
 (segment (start 54 150) (end 277 150) (width 8) (layer "B.Cu") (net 2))
 (segment (start 40.565482 109.862821) (end 41.179857 133.977019) (width 8) (layer "B.Cu") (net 2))
 (segment (start 57 90) (end 51.411765 90) (width 8) (layer "B.Cu") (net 2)))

